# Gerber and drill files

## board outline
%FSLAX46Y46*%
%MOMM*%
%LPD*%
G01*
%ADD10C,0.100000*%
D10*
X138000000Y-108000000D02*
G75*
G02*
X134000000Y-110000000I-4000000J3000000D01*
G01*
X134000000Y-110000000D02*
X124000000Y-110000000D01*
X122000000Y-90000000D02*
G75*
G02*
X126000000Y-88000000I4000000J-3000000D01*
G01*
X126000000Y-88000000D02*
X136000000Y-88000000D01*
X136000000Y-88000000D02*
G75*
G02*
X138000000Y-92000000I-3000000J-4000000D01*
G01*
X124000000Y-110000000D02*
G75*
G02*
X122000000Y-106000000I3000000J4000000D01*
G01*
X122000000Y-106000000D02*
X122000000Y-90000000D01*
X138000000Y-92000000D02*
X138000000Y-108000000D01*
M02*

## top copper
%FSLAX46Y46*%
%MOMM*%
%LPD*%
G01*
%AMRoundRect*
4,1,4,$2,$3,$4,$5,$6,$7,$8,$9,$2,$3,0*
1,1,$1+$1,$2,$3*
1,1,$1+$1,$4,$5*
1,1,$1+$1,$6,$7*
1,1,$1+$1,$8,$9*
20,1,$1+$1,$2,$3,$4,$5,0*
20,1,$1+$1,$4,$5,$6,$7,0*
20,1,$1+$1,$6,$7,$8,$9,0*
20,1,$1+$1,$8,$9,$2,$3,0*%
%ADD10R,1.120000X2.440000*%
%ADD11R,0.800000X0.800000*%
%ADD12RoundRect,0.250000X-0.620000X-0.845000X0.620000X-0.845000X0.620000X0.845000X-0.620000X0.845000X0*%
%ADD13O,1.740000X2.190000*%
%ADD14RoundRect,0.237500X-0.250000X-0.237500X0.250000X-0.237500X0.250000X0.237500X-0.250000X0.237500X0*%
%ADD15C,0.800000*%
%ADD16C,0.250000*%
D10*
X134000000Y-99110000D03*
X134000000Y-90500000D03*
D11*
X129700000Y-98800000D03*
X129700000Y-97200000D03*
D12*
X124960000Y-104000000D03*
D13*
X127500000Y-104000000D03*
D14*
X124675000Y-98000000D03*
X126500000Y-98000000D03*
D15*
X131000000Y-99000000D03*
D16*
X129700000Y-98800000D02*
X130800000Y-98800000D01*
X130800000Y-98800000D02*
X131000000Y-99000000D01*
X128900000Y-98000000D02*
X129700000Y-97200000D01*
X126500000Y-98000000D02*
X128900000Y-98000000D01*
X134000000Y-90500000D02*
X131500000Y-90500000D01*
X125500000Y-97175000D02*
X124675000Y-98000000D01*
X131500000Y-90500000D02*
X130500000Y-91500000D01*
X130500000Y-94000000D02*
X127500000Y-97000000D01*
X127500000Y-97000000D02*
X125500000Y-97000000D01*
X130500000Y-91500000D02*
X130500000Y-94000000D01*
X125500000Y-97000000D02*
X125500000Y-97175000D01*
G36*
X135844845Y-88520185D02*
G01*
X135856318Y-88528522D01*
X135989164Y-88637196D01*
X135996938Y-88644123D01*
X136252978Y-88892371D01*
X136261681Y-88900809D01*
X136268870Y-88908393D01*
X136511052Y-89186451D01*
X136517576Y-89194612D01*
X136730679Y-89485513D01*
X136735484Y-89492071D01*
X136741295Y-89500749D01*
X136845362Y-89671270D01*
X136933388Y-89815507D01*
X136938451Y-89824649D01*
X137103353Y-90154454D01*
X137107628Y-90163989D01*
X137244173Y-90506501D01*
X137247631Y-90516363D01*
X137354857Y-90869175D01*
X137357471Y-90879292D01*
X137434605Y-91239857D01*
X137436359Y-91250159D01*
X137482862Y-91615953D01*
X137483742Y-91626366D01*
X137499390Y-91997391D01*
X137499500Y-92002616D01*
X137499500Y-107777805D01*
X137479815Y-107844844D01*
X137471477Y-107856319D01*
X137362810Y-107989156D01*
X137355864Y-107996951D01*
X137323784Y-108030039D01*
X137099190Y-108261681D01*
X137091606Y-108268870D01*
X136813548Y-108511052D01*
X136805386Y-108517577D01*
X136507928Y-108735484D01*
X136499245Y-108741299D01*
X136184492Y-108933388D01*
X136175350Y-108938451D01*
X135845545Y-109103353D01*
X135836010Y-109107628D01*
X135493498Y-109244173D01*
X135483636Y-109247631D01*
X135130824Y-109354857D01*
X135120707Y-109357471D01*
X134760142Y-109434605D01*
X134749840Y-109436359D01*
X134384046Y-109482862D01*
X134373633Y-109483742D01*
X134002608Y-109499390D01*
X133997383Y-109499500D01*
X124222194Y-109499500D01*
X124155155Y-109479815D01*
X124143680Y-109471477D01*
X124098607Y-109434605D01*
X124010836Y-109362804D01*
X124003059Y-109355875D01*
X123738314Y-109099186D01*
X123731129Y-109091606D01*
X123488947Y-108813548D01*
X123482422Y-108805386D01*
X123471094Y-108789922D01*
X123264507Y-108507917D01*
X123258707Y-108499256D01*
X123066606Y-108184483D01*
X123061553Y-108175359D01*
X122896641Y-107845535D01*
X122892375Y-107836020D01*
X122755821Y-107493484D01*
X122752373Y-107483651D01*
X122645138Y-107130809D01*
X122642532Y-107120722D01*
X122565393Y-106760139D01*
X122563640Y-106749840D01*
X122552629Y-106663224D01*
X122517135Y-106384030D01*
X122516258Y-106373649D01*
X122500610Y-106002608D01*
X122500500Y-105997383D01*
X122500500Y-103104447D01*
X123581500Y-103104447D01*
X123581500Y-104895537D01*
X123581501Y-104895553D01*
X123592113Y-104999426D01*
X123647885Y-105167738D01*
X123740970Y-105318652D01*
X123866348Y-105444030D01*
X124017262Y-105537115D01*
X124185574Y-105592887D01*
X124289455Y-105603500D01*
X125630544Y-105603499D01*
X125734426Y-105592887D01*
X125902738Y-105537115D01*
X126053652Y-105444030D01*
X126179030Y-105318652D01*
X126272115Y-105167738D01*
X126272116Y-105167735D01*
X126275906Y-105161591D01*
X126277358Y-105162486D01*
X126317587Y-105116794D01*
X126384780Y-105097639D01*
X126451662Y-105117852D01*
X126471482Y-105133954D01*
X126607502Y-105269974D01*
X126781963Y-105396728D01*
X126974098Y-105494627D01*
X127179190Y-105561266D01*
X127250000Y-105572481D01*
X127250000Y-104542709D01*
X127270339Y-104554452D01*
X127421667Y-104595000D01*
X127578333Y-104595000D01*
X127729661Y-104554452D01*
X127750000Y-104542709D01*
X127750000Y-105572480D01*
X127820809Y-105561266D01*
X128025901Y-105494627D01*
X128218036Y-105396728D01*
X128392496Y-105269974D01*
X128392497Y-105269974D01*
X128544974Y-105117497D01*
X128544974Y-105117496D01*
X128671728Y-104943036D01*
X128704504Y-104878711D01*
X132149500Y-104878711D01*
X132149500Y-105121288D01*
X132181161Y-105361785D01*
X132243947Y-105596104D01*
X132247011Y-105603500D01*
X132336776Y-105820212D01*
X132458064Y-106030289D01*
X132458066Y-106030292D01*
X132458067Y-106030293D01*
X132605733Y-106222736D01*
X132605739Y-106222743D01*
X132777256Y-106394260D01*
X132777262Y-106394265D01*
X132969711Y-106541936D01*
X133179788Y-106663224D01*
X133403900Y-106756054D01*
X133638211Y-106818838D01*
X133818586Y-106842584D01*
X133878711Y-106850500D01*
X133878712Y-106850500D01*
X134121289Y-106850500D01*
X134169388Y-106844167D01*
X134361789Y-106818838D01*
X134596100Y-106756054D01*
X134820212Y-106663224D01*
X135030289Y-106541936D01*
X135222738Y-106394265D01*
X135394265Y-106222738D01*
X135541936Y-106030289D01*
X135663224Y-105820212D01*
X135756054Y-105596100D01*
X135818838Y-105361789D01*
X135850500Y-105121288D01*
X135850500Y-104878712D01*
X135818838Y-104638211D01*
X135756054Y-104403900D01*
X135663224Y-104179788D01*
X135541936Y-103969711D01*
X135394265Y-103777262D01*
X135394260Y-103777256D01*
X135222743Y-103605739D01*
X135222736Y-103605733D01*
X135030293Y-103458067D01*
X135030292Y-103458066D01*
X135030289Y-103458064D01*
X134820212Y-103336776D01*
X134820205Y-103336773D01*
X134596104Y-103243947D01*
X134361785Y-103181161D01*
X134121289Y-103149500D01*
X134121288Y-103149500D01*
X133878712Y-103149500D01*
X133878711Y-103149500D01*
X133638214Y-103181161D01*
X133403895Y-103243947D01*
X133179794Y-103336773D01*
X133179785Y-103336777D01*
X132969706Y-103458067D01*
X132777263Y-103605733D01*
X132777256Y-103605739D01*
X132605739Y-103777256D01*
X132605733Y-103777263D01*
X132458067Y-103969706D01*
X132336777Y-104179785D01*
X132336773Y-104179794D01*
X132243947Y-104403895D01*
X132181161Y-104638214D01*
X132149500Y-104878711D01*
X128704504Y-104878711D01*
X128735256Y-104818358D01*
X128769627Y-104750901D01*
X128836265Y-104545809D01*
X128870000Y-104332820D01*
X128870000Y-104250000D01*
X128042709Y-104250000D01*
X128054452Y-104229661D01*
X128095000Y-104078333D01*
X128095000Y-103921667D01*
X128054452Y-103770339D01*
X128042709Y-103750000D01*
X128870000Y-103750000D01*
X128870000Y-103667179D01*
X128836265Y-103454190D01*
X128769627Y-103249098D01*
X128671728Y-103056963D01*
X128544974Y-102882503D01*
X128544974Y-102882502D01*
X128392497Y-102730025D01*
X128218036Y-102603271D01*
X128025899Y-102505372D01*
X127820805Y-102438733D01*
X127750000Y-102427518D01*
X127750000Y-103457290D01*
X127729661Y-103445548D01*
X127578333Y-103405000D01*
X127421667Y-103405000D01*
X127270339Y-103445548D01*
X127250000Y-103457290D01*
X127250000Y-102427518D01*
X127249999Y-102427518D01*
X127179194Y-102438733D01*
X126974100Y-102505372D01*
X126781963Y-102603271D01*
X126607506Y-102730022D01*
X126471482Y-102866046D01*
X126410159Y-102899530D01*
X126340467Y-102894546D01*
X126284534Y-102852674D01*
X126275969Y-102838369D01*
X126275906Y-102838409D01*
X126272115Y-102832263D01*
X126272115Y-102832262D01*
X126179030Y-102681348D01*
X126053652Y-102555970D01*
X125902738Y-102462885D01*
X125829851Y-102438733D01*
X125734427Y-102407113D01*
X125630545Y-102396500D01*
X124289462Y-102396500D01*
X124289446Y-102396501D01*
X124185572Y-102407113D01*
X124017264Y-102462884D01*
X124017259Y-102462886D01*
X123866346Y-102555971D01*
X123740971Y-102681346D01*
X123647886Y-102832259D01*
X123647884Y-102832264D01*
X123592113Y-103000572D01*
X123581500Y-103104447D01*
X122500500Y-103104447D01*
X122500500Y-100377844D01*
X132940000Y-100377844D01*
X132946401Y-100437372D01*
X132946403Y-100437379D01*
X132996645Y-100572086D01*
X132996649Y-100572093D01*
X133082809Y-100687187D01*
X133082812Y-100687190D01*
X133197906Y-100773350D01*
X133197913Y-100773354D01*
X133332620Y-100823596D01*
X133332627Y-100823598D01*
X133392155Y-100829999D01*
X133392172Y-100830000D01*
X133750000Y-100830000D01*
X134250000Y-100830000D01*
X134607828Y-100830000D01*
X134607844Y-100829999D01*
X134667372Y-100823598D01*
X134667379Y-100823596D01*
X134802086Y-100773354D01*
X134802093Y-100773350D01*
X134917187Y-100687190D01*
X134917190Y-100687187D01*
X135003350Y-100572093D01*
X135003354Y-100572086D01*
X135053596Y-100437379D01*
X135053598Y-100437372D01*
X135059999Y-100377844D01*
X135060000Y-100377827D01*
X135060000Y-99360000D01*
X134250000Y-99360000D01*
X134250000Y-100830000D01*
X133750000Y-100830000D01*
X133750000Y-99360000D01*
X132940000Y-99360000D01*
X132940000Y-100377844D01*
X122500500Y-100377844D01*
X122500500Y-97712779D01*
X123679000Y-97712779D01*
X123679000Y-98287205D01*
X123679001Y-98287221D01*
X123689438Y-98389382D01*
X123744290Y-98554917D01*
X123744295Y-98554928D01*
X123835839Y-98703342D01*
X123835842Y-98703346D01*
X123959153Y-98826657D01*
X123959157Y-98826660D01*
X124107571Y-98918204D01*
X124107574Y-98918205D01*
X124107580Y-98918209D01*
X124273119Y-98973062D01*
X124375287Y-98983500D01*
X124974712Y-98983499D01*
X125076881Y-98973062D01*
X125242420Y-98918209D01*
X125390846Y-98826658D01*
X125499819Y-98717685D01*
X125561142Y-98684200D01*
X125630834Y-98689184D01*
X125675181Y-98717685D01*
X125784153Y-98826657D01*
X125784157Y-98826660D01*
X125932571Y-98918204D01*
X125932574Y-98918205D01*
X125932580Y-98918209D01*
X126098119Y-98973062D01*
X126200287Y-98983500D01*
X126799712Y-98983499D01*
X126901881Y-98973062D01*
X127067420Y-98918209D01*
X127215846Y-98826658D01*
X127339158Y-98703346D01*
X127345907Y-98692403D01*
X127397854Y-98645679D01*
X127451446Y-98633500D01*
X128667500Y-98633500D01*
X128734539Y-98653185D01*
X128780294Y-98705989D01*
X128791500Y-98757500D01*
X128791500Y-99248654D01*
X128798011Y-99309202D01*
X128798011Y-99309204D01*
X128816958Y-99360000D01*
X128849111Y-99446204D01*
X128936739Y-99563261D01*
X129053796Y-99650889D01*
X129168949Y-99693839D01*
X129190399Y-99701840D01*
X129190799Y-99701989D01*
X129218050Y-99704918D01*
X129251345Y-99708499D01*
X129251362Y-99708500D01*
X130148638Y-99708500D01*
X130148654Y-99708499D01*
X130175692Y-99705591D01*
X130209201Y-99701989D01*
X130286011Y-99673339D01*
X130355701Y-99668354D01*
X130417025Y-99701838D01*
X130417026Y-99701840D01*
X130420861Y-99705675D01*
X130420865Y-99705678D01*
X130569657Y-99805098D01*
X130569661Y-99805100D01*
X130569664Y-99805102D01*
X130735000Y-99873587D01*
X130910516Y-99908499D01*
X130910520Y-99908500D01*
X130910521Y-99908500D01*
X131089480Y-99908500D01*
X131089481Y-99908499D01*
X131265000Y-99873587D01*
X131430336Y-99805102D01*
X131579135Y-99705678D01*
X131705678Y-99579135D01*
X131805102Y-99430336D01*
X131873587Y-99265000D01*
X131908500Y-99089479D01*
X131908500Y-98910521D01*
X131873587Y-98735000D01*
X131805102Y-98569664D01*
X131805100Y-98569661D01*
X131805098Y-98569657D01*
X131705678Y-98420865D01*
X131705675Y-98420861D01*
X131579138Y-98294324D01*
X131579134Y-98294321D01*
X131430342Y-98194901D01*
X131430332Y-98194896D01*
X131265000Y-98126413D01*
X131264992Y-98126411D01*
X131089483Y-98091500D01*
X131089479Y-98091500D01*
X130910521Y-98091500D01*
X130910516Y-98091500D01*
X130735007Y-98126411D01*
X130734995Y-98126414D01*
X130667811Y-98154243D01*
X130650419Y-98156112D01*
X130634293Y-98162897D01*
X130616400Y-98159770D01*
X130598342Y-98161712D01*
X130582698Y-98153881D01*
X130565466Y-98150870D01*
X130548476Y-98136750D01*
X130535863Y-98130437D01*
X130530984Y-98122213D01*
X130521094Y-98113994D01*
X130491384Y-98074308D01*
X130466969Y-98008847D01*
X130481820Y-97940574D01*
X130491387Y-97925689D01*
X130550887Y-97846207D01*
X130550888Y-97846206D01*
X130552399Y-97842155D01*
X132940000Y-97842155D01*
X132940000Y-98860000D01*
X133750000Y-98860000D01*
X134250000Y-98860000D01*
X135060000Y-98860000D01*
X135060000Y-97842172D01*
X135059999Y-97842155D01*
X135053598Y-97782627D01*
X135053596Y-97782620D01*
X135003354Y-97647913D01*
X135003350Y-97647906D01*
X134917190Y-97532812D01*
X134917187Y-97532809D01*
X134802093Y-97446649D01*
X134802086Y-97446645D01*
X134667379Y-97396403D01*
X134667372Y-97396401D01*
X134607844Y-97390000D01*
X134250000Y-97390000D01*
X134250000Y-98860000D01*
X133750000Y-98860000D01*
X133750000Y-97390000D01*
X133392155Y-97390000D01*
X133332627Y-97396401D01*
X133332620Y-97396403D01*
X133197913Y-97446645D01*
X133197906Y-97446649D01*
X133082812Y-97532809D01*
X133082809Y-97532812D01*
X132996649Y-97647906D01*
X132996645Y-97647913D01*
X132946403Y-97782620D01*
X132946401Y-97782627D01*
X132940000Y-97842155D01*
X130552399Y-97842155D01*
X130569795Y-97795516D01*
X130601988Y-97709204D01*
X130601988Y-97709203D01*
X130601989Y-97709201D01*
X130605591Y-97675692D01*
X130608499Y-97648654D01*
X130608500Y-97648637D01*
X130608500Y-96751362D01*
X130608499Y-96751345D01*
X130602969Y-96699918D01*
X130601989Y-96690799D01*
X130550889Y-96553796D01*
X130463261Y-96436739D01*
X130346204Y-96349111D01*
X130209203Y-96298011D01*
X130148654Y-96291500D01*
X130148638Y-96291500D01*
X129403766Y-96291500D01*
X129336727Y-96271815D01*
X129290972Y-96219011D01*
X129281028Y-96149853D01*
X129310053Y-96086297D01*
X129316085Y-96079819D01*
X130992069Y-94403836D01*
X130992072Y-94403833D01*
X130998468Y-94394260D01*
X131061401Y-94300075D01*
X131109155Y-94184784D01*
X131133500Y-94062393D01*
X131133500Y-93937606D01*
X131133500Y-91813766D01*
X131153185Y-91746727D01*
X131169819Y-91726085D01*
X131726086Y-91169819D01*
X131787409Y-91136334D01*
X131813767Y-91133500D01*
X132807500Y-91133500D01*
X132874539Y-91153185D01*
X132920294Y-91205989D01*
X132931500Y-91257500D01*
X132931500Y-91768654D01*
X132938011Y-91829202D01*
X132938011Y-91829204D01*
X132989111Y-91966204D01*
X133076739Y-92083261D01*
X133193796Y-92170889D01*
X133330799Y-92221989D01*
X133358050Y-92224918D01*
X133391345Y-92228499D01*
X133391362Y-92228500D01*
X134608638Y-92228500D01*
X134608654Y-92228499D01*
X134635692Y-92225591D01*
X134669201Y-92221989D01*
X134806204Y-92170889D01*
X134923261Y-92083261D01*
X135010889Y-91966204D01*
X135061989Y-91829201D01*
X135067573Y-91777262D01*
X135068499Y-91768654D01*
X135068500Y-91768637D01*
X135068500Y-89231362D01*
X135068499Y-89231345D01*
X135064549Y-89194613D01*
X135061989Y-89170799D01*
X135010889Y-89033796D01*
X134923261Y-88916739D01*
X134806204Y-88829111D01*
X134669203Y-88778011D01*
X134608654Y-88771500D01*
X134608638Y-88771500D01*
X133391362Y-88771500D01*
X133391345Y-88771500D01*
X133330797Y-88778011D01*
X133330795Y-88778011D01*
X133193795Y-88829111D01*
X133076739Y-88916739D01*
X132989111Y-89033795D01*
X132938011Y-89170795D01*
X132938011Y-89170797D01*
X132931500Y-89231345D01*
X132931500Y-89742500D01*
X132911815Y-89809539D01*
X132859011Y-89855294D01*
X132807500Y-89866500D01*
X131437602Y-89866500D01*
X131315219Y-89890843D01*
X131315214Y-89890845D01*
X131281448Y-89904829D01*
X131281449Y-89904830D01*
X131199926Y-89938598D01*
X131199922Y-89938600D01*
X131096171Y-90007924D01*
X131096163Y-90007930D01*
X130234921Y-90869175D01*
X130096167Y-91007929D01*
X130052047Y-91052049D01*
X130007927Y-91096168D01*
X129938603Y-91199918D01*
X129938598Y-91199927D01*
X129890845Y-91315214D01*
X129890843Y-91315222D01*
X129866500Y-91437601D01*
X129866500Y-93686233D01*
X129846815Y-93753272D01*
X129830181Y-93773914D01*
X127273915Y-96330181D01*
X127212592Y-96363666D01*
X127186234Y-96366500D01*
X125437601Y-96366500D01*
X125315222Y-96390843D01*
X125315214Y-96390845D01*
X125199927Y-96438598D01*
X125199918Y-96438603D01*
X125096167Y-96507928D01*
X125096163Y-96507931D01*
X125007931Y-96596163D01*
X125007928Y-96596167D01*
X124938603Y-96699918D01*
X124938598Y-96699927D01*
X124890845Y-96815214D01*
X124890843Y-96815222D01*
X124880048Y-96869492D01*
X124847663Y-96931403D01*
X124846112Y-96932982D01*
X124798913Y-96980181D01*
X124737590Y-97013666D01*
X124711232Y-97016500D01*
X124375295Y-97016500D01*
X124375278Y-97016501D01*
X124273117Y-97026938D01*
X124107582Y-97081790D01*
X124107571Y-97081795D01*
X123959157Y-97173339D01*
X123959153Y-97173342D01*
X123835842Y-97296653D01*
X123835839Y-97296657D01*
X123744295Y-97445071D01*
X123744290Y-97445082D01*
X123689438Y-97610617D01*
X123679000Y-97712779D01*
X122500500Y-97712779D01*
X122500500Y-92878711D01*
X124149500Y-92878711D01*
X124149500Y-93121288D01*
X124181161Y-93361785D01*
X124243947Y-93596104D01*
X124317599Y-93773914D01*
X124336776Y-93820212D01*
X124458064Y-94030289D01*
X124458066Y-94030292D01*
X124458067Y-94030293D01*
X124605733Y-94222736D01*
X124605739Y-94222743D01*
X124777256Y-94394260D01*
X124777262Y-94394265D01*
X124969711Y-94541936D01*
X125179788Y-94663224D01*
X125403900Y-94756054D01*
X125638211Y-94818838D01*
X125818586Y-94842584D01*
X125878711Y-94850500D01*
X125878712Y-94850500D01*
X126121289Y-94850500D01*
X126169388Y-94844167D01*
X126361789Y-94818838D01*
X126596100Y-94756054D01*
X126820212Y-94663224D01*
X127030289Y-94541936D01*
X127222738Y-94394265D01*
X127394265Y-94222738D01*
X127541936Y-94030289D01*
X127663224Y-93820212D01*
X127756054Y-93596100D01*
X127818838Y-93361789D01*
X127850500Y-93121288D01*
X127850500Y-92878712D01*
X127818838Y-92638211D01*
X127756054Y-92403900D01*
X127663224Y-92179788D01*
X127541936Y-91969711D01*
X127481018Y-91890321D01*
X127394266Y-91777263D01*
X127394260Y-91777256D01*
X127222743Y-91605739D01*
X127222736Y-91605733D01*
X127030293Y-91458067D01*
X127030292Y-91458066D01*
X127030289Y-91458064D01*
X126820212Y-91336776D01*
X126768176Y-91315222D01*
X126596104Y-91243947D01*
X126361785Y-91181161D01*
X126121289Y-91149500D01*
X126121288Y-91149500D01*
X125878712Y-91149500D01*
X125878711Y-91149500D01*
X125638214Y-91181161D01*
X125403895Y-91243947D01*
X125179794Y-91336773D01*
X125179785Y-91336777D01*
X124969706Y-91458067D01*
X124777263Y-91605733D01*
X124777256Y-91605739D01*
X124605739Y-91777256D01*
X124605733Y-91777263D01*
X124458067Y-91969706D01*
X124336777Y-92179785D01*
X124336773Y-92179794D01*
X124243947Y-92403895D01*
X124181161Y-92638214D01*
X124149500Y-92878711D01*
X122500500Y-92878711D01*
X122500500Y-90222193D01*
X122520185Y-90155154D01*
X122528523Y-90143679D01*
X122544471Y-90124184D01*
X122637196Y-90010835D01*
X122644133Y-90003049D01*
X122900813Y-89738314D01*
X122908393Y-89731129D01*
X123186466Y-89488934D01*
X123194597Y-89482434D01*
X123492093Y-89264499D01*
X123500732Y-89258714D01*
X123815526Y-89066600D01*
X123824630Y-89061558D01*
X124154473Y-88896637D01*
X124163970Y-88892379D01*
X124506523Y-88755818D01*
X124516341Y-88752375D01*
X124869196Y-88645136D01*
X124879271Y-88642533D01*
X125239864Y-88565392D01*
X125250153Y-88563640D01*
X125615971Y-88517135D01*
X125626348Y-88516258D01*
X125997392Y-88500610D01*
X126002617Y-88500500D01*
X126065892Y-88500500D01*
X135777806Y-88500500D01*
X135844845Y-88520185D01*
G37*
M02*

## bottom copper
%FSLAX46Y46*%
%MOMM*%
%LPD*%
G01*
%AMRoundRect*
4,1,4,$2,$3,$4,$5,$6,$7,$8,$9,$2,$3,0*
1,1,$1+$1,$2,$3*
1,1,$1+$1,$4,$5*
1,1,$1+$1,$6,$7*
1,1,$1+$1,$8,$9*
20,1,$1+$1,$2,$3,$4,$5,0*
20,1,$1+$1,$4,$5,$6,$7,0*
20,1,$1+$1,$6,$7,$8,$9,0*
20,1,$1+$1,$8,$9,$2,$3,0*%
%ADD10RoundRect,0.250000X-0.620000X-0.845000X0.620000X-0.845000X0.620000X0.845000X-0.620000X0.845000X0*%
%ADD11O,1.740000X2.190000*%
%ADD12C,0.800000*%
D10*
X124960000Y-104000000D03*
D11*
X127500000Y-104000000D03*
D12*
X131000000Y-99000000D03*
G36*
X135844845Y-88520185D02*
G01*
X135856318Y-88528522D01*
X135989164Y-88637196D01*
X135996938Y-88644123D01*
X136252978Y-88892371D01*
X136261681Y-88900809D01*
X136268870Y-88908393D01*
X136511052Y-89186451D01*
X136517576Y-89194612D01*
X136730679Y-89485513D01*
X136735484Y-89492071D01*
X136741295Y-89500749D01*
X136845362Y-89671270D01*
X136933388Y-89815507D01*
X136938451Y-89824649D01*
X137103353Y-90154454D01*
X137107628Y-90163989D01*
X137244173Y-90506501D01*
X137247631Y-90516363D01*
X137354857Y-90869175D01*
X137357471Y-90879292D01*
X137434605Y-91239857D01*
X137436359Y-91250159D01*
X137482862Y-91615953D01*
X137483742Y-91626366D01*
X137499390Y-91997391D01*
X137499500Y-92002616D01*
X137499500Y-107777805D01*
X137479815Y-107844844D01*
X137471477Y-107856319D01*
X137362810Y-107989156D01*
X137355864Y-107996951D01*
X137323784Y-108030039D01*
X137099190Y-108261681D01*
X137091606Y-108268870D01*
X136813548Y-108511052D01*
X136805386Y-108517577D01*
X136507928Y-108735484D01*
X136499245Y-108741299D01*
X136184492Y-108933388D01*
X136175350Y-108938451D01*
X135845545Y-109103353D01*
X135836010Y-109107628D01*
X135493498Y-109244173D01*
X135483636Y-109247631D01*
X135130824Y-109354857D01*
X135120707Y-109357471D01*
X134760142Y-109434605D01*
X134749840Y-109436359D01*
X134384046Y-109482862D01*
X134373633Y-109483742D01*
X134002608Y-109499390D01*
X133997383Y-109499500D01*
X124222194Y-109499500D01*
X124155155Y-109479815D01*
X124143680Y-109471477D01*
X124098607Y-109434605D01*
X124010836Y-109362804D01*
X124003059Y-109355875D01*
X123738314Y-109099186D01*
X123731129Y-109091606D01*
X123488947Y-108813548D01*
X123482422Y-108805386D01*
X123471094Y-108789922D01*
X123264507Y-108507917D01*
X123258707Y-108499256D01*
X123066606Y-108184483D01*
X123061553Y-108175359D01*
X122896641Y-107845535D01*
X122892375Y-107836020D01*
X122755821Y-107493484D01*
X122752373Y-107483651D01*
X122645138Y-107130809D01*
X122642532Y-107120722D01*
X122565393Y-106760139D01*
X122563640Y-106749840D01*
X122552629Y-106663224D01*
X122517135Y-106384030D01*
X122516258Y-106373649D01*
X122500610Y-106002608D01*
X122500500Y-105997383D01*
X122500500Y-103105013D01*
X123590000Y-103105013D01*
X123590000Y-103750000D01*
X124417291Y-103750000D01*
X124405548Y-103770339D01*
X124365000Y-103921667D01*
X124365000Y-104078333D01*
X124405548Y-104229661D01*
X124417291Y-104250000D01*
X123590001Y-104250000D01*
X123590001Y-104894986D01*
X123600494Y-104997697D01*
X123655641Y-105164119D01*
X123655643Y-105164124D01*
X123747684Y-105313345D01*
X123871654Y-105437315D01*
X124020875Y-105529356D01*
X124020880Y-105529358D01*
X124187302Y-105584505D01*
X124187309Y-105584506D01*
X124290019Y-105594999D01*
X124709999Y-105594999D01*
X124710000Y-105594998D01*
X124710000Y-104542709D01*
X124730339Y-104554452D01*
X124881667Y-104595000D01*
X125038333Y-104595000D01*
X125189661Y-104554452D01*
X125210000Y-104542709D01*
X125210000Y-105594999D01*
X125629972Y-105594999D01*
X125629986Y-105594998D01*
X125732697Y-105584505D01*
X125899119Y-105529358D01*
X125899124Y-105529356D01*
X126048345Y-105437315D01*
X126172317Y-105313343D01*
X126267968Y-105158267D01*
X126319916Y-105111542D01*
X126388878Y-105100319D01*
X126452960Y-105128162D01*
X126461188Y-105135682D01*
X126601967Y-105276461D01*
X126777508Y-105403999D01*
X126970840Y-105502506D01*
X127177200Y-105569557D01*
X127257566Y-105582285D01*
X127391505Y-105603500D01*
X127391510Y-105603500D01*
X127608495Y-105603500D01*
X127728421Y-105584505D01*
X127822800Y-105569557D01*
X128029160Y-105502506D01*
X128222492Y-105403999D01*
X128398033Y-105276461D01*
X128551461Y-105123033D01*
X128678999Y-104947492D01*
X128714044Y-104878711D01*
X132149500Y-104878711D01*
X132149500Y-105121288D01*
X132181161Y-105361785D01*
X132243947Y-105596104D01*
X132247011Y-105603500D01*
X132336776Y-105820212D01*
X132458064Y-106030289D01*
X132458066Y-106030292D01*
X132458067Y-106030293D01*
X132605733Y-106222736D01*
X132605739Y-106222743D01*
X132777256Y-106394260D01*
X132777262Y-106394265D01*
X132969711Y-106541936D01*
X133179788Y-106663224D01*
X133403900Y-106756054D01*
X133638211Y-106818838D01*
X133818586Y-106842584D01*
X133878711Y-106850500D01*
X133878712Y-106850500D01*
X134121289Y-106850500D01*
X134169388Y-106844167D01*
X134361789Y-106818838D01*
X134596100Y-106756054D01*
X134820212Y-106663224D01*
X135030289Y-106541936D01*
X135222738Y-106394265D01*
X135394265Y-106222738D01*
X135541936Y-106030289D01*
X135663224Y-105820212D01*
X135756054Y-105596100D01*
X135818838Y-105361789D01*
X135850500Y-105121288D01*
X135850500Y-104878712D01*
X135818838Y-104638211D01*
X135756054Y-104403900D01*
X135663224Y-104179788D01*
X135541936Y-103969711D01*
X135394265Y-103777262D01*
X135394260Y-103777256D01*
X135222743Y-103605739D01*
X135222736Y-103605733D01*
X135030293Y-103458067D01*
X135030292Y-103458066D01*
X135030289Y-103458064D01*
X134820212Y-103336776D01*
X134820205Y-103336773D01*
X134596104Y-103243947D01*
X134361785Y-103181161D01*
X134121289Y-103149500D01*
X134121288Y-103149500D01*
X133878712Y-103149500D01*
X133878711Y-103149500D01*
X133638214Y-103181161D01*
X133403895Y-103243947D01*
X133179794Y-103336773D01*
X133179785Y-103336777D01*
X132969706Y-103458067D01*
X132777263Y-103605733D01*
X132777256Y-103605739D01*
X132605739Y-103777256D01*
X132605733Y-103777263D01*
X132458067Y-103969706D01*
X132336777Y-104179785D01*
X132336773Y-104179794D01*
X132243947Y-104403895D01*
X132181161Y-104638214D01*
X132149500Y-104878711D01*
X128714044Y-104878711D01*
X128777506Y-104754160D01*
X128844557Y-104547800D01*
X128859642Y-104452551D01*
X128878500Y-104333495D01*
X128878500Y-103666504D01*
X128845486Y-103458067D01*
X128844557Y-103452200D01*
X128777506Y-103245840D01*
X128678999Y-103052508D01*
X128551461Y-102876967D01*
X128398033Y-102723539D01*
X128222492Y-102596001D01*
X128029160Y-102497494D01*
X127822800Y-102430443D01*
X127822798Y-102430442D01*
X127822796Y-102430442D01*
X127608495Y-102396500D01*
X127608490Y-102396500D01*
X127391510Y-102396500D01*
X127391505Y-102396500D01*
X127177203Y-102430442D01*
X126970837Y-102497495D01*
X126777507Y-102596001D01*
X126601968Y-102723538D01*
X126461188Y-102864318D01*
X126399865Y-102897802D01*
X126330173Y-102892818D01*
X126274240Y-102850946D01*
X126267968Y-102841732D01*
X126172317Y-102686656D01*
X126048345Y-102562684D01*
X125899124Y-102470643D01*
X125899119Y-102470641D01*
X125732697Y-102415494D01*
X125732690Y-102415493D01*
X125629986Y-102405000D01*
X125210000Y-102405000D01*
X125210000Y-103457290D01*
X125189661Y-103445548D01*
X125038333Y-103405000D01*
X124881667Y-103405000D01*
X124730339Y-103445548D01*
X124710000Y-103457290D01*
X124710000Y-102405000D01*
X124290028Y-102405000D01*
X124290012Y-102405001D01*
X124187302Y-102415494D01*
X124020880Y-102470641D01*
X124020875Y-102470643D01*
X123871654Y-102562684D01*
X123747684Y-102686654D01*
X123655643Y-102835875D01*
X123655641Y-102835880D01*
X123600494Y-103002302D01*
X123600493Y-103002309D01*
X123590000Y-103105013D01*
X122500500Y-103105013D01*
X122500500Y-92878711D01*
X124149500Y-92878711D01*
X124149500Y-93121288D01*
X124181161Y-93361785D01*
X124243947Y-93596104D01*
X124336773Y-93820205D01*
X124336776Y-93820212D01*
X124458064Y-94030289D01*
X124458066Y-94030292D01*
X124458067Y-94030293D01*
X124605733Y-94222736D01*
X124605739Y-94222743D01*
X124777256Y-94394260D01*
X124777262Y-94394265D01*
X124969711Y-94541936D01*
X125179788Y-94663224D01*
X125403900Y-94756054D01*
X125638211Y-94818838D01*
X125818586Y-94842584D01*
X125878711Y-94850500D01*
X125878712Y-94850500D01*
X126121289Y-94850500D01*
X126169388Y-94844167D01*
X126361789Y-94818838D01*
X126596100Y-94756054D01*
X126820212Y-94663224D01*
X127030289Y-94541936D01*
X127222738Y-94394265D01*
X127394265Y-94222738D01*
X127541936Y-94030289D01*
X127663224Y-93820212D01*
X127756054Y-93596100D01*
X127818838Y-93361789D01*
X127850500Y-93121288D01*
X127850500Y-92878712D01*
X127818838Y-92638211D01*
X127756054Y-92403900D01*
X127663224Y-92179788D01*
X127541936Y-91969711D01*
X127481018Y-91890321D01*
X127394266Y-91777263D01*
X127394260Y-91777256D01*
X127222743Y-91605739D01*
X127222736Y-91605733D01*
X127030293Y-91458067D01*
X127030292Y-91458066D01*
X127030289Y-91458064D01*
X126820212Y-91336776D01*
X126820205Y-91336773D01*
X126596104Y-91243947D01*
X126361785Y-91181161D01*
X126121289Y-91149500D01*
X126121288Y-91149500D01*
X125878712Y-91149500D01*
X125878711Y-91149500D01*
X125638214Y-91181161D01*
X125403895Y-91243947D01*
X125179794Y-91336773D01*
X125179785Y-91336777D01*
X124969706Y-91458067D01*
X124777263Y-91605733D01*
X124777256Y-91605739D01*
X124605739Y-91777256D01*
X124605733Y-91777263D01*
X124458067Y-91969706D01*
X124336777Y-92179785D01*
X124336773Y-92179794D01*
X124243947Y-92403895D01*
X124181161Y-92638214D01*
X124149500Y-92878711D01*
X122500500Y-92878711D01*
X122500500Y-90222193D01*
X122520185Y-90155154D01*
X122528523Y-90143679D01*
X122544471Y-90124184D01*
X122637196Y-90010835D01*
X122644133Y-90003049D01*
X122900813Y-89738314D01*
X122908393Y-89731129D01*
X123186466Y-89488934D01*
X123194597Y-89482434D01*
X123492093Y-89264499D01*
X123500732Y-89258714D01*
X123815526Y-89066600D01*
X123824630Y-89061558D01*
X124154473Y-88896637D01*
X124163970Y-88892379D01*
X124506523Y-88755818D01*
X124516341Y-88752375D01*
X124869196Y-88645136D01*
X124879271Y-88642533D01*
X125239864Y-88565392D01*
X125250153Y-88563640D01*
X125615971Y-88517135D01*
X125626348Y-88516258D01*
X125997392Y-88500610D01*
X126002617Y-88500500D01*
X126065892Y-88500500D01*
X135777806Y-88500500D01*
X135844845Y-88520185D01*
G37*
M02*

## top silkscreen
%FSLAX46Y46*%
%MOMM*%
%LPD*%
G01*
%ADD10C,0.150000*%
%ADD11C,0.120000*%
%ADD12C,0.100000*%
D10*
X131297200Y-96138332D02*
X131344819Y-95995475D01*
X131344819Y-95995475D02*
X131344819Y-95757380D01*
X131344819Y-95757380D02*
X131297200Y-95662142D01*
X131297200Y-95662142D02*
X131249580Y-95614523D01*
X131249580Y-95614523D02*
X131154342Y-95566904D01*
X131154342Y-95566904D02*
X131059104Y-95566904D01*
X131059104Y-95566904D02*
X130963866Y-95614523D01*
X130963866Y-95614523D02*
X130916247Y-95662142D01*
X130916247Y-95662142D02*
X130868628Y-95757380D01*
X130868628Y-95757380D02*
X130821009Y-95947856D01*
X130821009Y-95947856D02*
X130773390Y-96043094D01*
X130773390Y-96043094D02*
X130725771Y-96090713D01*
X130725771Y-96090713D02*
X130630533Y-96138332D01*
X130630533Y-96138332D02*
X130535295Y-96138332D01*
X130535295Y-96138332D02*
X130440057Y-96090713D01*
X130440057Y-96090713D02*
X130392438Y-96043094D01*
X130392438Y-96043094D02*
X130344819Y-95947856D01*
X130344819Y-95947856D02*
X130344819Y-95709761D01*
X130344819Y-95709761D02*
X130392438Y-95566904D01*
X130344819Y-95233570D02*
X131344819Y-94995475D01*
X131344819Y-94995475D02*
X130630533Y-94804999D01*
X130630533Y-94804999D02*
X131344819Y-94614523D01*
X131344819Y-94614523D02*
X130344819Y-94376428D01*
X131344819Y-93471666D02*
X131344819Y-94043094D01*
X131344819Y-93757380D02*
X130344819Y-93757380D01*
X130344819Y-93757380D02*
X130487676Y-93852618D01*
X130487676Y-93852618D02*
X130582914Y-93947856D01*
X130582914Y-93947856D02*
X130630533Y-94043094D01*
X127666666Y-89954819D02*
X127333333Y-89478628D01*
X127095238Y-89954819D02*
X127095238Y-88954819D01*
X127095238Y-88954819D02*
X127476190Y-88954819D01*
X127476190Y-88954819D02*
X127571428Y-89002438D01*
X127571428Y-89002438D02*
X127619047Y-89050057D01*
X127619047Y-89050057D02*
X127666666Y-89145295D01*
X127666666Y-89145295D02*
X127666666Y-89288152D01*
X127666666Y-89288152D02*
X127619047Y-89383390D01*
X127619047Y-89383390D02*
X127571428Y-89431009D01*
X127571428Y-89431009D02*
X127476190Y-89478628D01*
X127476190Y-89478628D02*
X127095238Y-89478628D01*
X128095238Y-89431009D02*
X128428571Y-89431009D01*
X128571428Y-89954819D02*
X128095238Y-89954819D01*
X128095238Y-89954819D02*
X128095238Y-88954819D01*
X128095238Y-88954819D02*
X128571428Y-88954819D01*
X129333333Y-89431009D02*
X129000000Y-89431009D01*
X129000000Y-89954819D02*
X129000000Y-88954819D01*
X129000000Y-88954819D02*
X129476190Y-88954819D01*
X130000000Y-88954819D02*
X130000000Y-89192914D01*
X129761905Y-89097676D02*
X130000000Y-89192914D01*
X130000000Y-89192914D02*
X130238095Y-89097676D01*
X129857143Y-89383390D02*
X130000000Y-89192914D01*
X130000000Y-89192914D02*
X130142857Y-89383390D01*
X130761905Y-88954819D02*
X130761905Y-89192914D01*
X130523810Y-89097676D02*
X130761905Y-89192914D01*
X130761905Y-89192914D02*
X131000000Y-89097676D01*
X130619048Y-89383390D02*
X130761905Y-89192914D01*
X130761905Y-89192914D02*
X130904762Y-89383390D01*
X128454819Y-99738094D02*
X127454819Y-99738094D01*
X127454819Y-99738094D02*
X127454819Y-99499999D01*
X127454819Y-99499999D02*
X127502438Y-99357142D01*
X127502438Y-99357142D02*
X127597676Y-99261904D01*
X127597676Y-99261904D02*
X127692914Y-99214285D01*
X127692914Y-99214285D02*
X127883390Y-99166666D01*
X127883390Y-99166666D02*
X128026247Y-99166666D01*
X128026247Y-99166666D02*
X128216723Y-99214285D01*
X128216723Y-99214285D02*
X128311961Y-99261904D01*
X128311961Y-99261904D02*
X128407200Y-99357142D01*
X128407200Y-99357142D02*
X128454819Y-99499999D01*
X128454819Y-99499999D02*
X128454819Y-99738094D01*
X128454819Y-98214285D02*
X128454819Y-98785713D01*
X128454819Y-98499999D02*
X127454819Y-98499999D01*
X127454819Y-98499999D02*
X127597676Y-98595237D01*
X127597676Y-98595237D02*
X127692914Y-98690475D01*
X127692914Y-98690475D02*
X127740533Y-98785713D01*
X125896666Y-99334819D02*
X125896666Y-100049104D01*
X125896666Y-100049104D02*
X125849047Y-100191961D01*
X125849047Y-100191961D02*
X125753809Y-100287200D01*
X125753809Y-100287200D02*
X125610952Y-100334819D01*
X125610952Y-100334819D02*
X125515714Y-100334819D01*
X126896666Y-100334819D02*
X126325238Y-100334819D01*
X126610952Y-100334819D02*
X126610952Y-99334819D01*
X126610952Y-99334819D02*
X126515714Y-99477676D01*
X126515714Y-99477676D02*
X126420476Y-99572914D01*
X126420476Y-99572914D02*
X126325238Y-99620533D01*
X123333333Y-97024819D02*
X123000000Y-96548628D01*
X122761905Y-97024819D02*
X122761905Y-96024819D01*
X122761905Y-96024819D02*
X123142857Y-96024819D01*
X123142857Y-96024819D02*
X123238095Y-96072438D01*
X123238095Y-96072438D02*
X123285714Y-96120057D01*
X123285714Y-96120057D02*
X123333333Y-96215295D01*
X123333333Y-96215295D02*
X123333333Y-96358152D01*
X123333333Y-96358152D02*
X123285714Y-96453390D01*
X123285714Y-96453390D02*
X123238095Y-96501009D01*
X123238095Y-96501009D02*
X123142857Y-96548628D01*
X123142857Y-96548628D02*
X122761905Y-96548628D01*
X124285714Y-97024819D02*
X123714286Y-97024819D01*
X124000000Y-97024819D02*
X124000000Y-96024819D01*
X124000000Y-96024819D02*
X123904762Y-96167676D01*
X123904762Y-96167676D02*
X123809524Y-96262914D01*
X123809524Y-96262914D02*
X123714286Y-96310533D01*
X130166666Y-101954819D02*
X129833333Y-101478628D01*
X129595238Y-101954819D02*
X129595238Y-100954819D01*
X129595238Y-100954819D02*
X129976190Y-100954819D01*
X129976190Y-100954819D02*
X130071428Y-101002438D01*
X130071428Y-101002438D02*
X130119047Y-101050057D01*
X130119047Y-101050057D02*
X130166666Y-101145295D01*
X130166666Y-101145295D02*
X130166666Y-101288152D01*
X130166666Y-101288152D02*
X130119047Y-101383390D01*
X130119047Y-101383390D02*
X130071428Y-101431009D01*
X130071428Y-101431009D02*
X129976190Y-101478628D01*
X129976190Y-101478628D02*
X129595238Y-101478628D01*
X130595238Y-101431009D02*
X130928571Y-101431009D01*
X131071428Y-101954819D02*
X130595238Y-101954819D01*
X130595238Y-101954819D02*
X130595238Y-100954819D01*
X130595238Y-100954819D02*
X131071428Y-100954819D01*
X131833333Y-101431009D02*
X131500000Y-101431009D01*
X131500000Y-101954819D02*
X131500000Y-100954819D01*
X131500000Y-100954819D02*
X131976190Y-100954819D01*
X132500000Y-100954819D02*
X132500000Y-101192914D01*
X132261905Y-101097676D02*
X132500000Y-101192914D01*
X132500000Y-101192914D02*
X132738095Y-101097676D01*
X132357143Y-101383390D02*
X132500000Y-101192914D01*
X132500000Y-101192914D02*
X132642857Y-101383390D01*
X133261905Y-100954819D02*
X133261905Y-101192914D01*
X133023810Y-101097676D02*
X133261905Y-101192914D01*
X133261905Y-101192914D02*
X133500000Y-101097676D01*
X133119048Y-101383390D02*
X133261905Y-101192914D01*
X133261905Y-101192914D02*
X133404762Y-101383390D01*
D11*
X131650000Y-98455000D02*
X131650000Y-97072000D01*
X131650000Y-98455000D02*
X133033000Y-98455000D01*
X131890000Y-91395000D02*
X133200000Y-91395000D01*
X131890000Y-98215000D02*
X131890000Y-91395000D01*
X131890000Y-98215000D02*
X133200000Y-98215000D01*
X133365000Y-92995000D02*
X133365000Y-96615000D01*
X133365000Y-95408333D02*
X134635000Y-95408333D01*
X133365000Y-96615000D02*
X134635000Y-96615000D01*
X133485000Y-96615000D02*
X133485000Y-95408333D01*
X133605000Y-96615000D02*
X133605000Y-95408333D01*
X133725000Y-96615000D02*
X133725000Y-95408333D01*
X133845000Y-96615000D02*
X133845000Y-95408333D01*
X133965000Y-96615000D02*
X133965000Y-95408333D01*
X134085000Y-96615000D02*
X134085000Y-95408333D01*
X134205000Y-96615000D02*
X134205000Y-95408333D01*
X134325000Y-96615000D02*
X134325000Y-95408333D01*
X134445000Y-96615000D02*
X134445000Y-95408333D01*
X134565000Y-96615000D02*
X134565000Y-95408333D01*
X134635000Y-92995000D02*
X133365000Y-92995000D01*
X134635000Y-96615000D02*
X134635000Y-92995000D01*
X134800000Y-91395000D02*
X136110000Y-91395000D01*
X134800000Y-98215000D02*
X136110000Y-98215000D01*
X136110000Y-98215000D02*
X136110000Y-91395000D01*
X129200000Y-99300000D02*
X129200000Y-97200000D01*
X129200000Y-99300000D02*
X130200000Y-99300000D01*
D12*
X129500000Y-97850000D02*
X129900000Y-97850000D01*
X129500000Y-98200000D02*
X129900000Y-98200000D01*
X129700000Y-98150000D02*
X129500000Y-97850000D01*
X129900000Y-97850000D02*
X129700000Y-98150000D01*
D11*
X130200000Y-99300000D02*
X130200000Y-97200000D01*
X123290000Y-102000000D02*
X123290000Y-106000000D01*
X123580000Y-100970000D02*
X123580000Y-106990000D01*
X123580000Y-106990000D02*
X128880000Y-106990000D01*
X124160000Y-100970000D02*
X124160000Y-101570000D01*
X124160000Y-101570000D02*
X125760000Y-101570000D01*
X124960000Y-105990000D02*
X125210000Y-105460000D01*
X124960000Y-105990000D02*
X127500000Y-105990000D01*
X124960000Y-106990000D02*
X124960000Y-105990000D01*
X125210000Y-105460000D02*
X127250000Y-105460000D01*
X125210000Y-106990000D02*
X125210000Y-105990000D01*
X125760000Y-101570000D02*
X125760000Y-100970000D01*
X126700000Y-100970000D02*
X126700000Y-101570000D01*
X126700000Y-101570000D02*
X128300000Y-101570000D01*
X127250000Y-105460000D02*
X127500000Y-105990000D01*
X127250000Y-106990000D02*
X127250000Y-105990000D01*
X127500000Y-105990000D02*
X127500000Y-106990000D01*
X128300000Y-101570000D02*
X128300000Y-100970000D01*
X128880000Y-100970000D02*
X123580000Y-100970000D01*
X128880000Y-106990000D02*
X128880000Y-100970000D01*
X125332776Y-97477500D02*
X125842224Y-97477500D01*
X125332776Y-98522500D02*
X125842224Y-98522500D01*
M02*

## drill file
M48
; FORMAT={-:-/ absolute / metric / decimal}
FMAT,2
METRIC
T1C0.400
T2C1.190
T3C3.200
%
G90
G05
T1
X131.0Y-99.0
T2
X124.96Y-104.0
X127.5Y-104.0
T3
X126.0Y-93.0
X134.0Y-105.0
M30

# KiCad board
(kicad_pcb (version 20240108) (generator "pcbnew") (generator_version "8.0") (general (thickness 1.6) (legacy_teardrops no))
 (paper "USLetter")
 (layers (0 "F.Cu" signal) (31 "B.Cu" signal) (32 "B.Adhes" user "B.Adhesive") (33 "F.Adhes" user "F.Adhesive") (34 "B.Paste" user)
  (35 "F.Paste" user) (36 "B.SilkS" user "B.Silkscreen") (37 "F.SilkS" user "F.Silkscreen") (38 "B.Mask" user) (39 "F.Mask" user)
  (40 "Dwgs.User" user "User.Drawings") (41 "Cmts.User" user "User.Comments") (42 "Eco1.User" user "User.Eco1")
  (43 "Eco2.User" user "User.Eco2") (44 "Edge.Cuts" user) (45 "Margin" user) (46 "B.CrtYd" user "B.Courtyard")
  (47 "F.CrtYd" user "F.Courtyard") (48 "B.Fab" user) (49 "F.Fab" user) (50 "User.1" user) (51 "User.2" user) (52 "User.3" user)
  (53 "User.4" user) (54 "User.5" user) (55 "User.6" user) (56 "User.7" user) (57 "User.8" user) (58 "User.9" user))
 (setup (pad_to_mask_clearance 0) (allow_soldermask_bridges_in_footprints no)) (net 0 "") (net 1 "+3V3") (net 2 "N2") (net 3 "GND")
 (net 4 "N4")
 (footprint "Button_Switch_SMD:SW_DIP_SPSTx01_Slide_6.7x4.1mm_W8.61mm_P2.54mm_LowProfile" (layer "F.Cu") (at 134 94.805 90)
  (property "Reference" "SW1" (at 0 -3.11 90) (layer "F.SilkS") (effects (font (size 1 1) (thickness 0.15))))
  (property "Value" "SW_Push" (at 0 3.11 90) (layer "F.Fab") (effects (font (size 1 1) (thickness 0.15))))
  (fp_line (start -3.65 -2.35) (end -2.267 -2.35) (stroke (width 0.12) (type solid)) (layer "F.SilkS"))
  (fp_line (start -3.65 -2.35) (end -3.65 -0.967) (stroke (width 0.12) (type solid)) (layer "F.SilkS"))
  (fp_line (start 3.41 -2.11) (end 3.41 -0.8) (stroke (width 0.12) (type solid)) (layer "F.SilkS"))
  (fp_line (start -3.41 -2.11) (end 3.41 -2.11) (stroke (width 0.12) (type solid)) (layer "F.SilkS"))
  (fp_line (start -3.41 -2.11) (end -3.41 -0.8) (stroke (width 0.12) (type solid)) (layer "F.SilkS"))
  (fp_line (start 1.81 -0.635) (end -1.81 -0.635) (stroke (width 0.12) (type solid)) (layer "F.SilkS"))
  (fp_line (start -0.603333 -0.635) (end -0.603333 0.635) (stroke (width 0.12) (type solid)) (layer "F.SilkS"))
  (fp_line (start -1.81 -0.635) (end -1.81 0.635) (stroke (width 0.12) (type solid)) (layer "F.SilkS"))
  (fp_line (start -1.81 -0.515) (end -0.603333 -0.515) (stroke (width 0.12) (type solid)) (layer "F.SilkS"))
  (fp_line (start -1.81 -0.395) (end -0.603333 -0.395) (stroke (width 0.12) (type solid)) (layer "F.SilkS"))
  (fp_line (start -1.81 -0.275) (end -0.603333 -0.275) (stroke (width 0.12) (type solid)) (layer "F.SilkS"))
  (fp_line (start -1.81 -0.155) (end -0.603333 -0.155) (stroke (width 0.12) (type solid)) (layer "F.SilkS"))
  (fp_line (start -1.81 -0.035) (end -0.603333 -0.035) (stroke (width 0.12) (type solid)) (layer "F.SilkS"))
  (fp_line (start -1.81 0.085) (end -0.603333 0.085) (stroke (width 0.12) (type solid)) (layer "F.SilkS"))
  (fp_line (start -1.81 0.205) (end -0.603333 0.205) (stroke (width 0.12) (type solid)) (layer "F.SilkS"))
  (fp_line (start -1.81 0.325) (end -0.603333 0.325) (stroke (width 0.12) (type solid)) (layer "F.SilkS"))
  (fp_line (start -1.81 0.445) (end -0.603333 0.445) (stroke (width 0.12) (type solid)) (layer "F.SilkS"))
  (fp_line (start -1.81 0.565) (end -0.603333 0.565) (stroke (width 0.12) (type solid)) (layer "F.SilkS"))
  (fp_line (start 1.81 0.635) (end 1.81 -0.635) (stroke (width 0.12) (type solid)) (layer "F.SilkS"))
  (fp_line (start -1.81 0.635) (end 1.81 0.635) (stroke (width 0.12) (type solid)) (layer "F.SilkS"))
  (fp_line (start 3.41 0.8) (end 3.41 2.11) (stroke (width 0.12) (type solid)) (layer "F.SilkS"))
  (fp_line (start -3.41 0.8) (end -3.41 2.11) (stroke (width 0.12) (type solid)) (layer "F.SilkS"))
  (fp_line (start -3.41 2.11) (end 3.41 2.11) (stroke (width 0.12) (type solid)) (layer "F.SilkS"))
  (pad "1" smd rect (at -4.305 0 90) (size 2.44 1.12) (layers "F.Cu" "F.Paste" "F.Mask") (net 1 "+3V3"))
  (pad "2" smd rect (at 4.305 0 90) (size 2.44 1.12) (layers "F.Cu" "F.Paste" "F.Mask") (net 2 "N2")))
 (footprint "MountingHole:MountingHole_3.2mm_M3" (layer "F.Cu") (at 126 93)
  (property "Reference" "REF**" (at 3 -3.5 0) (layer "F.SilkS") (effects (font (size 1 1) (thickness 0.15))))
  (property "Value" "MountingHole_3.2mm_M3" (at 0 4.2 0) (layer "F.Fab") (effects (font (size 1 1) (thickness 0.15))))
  (pad "" np_thru_hole circle (at 0 0) (size 3.2 3.2) (drill 3.2) (layers "*.Cu" "*.Mask")))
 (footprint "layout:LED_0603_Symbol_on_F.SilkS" (layer "F.Cu") (at 129.7 98 90)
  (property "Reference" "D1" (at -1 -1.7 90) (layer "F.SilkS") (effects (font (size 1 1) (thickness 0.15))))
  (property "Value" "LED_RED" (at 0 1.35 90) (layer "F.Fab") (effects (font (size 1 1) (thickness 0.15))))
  (fp_line (start -1.3 -0.5) (end 0.8 -0.5) (stroke (width 0.12) (type solid)) (layer "F.SilkS"))
  (fp_line (start -1.3 -0.5) (end -1.3 0.5) (stroke (width 0.12) (type solid)) (layer "F.SilkS"))
  (fp_line (start 0.15 -0.2) (end 0.15 0.2) (stroke (width 0.1) (type solid)) (layer "F.SilkS"))
  (fp_line (start -0.2 -0.2) (end -0.2 0.2) (stroke (width 0.1) (type solid)) (layer "F.SilkS"))
  (fp_line (start -0.15 0) (end 0.15 -0.2) (stroke (width 0.1) (type solid)) (layer "F.SilkS"))
  (fp_line (start 0.15 0.2) (end -0.15 0) (stroke (width 0.1) (type solid)) (layer "F.SilkS"))
  (fp_line (start -1.3 0.5) (end 0.8 0.5) (stroke (width 0.12) (type solid)) (layer "F.SilkS"))
  (pad "1" smd rect (at -0.8 0 270) (size 0.8 0.8) (layers "F.Cu" "F.Paste" "F.Mask") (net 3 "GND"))
  (pad "2" smd rect (at 0.8 0 270) (size 0.8 0.8) (layers "F.Cu" "F.Paste" "F.Mask") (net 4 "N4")))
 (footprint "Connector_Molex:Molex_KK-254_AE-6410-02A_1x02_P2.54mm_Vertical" (layer "F.Cu") (at 124.96 104)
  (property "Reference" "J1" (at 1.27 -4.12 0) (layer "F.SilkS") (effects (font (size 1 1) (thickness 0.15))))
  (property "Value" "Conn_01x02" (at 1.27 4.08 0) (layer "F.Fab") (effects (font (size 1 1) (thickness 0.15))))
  (fp_line (start -1.67 -2) (end -1.67 2) (stroke (width 0.12) (type solid)) (layer "F.SilkS"))
  (fp_line (start -1.38 -3.03) (end -1.38 2.99) (stroke (width 0.12) (type solid)) (layer "F.SilkS"))
  (fp_line (start -1.38 2.99) (end 3.92 2.99) (stroke (width 0.12) (type solid)) (layer "F.SilkS"))
  (fp_line (start -0.8 -3.03) (end -0.8 -2.43) (stroke (width 0.12) (type solid)) (layer "F.SilkS"))
  (fp_line (start -0.8 -2.43) (end 0.8 -2.43) (stroke (width 0.12) (type solid)) (layer "F.SilkS"))
  (fp_line (start 0 1.99) (end 0.25 1.46) (stroke (width 0.12) (type solid)) (layer "F.SilkS"))
  (fp_line (start 0 1.99) (end 2.54 1.99) (stroke (width 0.12) (type solid)) (layer "F.SilkS"))
  (fp_line (start 0 2.99) (end 0 1.99) (stroke (width 0.12) (type solid)) (layer "F.SilkS"))
  (fp_line (start 0.25 1.46) (end 2.29 1.46) (stroke (width 0.12) (type solid)) (layer "F.SilkS"))
  (fp_line (start 0.25 2.99) (end 0.25 1.99) (stroke (width 0.12) (type solid)) (layer "F.SilkS"))
  (fp_line (start 0.8 -2.43) (end 0.8 -3.03) (stroke (width 0.12) (type solid)) (layer "F.SilkS"))
  (fp_line (start 1.74 -3.03) (end 1.74 -2.43) (stroke (width 0.12) (type solid)) (layer "F.SilkS"))
  (fp_line (start 1.74 -2.43) (end 3.34 -2.43) (stroke (width 0.12) (type solid)) (layer "F.SilkS"))
  (fp_line (start 2.29 1.46) (end 2.54 1.99) (stroke (width 0.12) (type solid)) (layer "F.SilkS"))
  (fp_line (start 2.29 2.99) (end 2.29 1.99) (stroke (width 0.12) (type solid)) (layer "F.SilkS"))
  (fp_line (start 2.54 1.99) (end 2.54 2.99) (stroke (width 0.12) (type solid)) (layer "F.SilkS"))
  (fp_line (start 3.34 -2.43) (end 3.34 -3.03) (stroke (width 0.12) (type solid)) (layer "F.SilkS"))
  (fp_line (start 3.92 -3.03) (end -1.38 -3.03) (stroke (width 0.12) (type solid)) (layer "F.SilkS"))
  (fp_line (start 3.92 2.99) (end 3.92 -3.03) (stroke (width 0.12) (type solid)) (layer "F.SilkS"))
  (pad "1" thru_hole roundrect (at 0 0) (size 1.74 2.19) (drill 1.19) (layers "*.Cu" "*.Mask") (remove_unused_layers no)
   (roundrect_rratio 0.143678) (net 3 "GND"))
  (pad "2" thru_hole oval (at 2.54 0) (size 1.74 2.19) (drill 1.19) (layers "*.Cu" "*.Mask") (remove_unused_layers no) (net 1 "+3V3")))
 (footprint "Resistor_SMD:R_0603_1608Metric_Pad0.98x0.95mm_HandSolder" (layer "F.Cu") (at 125.5875 98)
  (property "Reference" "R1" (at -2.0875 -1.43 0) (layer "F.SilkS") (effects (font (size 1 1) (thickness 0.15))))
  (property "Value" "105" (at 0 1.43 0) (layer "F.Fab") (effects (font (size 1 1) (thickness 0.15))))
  (fp_line (start -0.254724 -0.5225) (end 0.254724 -0.5225) (stroke (width 0.12) (type solid)) (layer "F.SilkS"))
  (fp_line (start -0.254724 0.5225) (end 0.254724 0.5225) (stroke (width 0.12) (type solid)) (layer "F.SilkS"))
  (pad "1" smd roundrect (at -0.9125 0) (size 0.975 0.95) (layers "F.Cu" "F.Paste" "F.Mask") (roundrect_rratio 0.25) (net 2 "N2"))
  (pad "2" smd roundrect (at 0.9125 0) (size 0.975 0.95) (layers "F.Cu" "F.Paste" "F.Mask") (roundrect_rratio 0.25) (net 4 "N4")))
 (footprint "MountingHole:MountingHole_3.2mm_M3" (layer "F.Cu") (at 134 105)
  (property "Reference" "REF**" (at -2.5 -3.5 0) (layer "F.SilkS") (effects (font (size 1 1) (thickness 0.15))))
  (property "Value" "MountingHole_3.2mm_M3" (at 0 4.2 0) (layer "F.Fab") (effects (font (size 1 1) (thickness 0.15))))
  (pad "" np_thru_hole circle (at 0 0) (size 3.2 3.2) (drill 3.2) (layers "*.Cu" "*.Mask")))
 (gr_arc (start 138 108) (mid 136.236068 109.472136) (end 134 110) (stroke (width 0.1) (type default)) (layer "Edge.Cuts"))
 (gr_line (start 134 110) (end 124 110) (stroke (width 0.1) (type default)) (layer "Edge.Cuts"))
 (gr_arc (start 122 90) (mid 123.763932 88.527864) (end 126 88) (stroke (width 0.1) (type default)) (layer "Edge.Cuts"))
 (gr_line (start 126 88) (end 136 88) (stroke (width 0.1) (type default)) (layer "Edge.Cuts"))
 (gr_arc (start 136 88) (mid 137.472136 89.763932) (end 138 92) (stroke (width 0.1) (type default)) (layer "Edge.Cuts"))
 (gr_arc (start 124 110) (mid 122.527864 108.236068) (end 122 106) (stroke (width 0.1) (type default)) (layer "Edge.Cuts"))
 (gr_line (start 122 106) (end 122 90) (stroke (width 0.1) (type default)) (layer "Edge.Cuts"))
 (gr_line (start 138 92) (end 138 108) (stroke (width 0.1) (type default)) (layer "Edge.Cuts"))
 (segment (start 129.7 98.8) (end 130.8 98.8) (width 0.25) (layer "F.Cu") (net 3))
 (segment (start 130.8 98.8) (end 131 99) (width 0.25) (layer "F.Cu") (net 3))
 (via (at 131 99) (size 0.8) (drill 0.4) (layers "F.Cu" "B.Cu") (free yes) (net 3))
 (segment (start 128.9 98) (end 129.7 97.2) (width 0.25) (layer "F.Cu") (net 4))
 (segment (start 126.5 98) (end 128.9 98) (width 0.25) (layer "F.Cu") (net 4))
 (segment (start 134 90.5) (end 131.5 90.5) (width 0.25) (layer "F.Cu") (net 2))
 (segment (start 125.5 97.175) (end 124.675 98) (width 0.25) (layer "F.Cu") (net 2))
 (segment (start 131.5 90.5) (end 130.5 91.5) (width 0.25) (layer "F.Cu") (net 2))
 (segment (start 130.5 94) (end 127.5 97) (width 0.25) (layer "F.Cu") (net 2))
 (segment (start 127.5 97) (end 125.5 97) (width 0.25) (layer "F.Cu") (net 2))
 (segment (start 130.5 91.5) (end 130.5 94) (width 0.25) (layer "F.Cu") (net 2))
 (segment (start 125.5 97) (end 125.5 97.175) (width 0.25) (layer "F.Cu") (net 2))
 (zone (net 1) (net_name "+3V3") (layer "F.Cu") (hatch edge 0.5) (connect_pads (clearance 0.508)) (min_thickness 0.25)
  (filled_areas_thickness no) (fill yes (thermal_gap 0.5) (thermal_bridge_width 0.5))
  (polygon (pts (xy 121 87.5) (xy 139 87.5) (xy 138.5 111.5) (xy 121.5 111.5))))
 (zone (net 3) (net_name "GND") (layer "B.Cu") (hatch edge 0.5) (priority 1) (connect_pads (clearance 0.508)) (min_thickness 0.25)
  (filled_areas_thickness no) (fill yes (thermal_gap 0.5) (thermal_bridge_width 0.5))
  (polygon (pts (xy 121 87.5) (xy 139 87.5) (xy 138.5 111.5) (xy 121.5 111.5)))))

